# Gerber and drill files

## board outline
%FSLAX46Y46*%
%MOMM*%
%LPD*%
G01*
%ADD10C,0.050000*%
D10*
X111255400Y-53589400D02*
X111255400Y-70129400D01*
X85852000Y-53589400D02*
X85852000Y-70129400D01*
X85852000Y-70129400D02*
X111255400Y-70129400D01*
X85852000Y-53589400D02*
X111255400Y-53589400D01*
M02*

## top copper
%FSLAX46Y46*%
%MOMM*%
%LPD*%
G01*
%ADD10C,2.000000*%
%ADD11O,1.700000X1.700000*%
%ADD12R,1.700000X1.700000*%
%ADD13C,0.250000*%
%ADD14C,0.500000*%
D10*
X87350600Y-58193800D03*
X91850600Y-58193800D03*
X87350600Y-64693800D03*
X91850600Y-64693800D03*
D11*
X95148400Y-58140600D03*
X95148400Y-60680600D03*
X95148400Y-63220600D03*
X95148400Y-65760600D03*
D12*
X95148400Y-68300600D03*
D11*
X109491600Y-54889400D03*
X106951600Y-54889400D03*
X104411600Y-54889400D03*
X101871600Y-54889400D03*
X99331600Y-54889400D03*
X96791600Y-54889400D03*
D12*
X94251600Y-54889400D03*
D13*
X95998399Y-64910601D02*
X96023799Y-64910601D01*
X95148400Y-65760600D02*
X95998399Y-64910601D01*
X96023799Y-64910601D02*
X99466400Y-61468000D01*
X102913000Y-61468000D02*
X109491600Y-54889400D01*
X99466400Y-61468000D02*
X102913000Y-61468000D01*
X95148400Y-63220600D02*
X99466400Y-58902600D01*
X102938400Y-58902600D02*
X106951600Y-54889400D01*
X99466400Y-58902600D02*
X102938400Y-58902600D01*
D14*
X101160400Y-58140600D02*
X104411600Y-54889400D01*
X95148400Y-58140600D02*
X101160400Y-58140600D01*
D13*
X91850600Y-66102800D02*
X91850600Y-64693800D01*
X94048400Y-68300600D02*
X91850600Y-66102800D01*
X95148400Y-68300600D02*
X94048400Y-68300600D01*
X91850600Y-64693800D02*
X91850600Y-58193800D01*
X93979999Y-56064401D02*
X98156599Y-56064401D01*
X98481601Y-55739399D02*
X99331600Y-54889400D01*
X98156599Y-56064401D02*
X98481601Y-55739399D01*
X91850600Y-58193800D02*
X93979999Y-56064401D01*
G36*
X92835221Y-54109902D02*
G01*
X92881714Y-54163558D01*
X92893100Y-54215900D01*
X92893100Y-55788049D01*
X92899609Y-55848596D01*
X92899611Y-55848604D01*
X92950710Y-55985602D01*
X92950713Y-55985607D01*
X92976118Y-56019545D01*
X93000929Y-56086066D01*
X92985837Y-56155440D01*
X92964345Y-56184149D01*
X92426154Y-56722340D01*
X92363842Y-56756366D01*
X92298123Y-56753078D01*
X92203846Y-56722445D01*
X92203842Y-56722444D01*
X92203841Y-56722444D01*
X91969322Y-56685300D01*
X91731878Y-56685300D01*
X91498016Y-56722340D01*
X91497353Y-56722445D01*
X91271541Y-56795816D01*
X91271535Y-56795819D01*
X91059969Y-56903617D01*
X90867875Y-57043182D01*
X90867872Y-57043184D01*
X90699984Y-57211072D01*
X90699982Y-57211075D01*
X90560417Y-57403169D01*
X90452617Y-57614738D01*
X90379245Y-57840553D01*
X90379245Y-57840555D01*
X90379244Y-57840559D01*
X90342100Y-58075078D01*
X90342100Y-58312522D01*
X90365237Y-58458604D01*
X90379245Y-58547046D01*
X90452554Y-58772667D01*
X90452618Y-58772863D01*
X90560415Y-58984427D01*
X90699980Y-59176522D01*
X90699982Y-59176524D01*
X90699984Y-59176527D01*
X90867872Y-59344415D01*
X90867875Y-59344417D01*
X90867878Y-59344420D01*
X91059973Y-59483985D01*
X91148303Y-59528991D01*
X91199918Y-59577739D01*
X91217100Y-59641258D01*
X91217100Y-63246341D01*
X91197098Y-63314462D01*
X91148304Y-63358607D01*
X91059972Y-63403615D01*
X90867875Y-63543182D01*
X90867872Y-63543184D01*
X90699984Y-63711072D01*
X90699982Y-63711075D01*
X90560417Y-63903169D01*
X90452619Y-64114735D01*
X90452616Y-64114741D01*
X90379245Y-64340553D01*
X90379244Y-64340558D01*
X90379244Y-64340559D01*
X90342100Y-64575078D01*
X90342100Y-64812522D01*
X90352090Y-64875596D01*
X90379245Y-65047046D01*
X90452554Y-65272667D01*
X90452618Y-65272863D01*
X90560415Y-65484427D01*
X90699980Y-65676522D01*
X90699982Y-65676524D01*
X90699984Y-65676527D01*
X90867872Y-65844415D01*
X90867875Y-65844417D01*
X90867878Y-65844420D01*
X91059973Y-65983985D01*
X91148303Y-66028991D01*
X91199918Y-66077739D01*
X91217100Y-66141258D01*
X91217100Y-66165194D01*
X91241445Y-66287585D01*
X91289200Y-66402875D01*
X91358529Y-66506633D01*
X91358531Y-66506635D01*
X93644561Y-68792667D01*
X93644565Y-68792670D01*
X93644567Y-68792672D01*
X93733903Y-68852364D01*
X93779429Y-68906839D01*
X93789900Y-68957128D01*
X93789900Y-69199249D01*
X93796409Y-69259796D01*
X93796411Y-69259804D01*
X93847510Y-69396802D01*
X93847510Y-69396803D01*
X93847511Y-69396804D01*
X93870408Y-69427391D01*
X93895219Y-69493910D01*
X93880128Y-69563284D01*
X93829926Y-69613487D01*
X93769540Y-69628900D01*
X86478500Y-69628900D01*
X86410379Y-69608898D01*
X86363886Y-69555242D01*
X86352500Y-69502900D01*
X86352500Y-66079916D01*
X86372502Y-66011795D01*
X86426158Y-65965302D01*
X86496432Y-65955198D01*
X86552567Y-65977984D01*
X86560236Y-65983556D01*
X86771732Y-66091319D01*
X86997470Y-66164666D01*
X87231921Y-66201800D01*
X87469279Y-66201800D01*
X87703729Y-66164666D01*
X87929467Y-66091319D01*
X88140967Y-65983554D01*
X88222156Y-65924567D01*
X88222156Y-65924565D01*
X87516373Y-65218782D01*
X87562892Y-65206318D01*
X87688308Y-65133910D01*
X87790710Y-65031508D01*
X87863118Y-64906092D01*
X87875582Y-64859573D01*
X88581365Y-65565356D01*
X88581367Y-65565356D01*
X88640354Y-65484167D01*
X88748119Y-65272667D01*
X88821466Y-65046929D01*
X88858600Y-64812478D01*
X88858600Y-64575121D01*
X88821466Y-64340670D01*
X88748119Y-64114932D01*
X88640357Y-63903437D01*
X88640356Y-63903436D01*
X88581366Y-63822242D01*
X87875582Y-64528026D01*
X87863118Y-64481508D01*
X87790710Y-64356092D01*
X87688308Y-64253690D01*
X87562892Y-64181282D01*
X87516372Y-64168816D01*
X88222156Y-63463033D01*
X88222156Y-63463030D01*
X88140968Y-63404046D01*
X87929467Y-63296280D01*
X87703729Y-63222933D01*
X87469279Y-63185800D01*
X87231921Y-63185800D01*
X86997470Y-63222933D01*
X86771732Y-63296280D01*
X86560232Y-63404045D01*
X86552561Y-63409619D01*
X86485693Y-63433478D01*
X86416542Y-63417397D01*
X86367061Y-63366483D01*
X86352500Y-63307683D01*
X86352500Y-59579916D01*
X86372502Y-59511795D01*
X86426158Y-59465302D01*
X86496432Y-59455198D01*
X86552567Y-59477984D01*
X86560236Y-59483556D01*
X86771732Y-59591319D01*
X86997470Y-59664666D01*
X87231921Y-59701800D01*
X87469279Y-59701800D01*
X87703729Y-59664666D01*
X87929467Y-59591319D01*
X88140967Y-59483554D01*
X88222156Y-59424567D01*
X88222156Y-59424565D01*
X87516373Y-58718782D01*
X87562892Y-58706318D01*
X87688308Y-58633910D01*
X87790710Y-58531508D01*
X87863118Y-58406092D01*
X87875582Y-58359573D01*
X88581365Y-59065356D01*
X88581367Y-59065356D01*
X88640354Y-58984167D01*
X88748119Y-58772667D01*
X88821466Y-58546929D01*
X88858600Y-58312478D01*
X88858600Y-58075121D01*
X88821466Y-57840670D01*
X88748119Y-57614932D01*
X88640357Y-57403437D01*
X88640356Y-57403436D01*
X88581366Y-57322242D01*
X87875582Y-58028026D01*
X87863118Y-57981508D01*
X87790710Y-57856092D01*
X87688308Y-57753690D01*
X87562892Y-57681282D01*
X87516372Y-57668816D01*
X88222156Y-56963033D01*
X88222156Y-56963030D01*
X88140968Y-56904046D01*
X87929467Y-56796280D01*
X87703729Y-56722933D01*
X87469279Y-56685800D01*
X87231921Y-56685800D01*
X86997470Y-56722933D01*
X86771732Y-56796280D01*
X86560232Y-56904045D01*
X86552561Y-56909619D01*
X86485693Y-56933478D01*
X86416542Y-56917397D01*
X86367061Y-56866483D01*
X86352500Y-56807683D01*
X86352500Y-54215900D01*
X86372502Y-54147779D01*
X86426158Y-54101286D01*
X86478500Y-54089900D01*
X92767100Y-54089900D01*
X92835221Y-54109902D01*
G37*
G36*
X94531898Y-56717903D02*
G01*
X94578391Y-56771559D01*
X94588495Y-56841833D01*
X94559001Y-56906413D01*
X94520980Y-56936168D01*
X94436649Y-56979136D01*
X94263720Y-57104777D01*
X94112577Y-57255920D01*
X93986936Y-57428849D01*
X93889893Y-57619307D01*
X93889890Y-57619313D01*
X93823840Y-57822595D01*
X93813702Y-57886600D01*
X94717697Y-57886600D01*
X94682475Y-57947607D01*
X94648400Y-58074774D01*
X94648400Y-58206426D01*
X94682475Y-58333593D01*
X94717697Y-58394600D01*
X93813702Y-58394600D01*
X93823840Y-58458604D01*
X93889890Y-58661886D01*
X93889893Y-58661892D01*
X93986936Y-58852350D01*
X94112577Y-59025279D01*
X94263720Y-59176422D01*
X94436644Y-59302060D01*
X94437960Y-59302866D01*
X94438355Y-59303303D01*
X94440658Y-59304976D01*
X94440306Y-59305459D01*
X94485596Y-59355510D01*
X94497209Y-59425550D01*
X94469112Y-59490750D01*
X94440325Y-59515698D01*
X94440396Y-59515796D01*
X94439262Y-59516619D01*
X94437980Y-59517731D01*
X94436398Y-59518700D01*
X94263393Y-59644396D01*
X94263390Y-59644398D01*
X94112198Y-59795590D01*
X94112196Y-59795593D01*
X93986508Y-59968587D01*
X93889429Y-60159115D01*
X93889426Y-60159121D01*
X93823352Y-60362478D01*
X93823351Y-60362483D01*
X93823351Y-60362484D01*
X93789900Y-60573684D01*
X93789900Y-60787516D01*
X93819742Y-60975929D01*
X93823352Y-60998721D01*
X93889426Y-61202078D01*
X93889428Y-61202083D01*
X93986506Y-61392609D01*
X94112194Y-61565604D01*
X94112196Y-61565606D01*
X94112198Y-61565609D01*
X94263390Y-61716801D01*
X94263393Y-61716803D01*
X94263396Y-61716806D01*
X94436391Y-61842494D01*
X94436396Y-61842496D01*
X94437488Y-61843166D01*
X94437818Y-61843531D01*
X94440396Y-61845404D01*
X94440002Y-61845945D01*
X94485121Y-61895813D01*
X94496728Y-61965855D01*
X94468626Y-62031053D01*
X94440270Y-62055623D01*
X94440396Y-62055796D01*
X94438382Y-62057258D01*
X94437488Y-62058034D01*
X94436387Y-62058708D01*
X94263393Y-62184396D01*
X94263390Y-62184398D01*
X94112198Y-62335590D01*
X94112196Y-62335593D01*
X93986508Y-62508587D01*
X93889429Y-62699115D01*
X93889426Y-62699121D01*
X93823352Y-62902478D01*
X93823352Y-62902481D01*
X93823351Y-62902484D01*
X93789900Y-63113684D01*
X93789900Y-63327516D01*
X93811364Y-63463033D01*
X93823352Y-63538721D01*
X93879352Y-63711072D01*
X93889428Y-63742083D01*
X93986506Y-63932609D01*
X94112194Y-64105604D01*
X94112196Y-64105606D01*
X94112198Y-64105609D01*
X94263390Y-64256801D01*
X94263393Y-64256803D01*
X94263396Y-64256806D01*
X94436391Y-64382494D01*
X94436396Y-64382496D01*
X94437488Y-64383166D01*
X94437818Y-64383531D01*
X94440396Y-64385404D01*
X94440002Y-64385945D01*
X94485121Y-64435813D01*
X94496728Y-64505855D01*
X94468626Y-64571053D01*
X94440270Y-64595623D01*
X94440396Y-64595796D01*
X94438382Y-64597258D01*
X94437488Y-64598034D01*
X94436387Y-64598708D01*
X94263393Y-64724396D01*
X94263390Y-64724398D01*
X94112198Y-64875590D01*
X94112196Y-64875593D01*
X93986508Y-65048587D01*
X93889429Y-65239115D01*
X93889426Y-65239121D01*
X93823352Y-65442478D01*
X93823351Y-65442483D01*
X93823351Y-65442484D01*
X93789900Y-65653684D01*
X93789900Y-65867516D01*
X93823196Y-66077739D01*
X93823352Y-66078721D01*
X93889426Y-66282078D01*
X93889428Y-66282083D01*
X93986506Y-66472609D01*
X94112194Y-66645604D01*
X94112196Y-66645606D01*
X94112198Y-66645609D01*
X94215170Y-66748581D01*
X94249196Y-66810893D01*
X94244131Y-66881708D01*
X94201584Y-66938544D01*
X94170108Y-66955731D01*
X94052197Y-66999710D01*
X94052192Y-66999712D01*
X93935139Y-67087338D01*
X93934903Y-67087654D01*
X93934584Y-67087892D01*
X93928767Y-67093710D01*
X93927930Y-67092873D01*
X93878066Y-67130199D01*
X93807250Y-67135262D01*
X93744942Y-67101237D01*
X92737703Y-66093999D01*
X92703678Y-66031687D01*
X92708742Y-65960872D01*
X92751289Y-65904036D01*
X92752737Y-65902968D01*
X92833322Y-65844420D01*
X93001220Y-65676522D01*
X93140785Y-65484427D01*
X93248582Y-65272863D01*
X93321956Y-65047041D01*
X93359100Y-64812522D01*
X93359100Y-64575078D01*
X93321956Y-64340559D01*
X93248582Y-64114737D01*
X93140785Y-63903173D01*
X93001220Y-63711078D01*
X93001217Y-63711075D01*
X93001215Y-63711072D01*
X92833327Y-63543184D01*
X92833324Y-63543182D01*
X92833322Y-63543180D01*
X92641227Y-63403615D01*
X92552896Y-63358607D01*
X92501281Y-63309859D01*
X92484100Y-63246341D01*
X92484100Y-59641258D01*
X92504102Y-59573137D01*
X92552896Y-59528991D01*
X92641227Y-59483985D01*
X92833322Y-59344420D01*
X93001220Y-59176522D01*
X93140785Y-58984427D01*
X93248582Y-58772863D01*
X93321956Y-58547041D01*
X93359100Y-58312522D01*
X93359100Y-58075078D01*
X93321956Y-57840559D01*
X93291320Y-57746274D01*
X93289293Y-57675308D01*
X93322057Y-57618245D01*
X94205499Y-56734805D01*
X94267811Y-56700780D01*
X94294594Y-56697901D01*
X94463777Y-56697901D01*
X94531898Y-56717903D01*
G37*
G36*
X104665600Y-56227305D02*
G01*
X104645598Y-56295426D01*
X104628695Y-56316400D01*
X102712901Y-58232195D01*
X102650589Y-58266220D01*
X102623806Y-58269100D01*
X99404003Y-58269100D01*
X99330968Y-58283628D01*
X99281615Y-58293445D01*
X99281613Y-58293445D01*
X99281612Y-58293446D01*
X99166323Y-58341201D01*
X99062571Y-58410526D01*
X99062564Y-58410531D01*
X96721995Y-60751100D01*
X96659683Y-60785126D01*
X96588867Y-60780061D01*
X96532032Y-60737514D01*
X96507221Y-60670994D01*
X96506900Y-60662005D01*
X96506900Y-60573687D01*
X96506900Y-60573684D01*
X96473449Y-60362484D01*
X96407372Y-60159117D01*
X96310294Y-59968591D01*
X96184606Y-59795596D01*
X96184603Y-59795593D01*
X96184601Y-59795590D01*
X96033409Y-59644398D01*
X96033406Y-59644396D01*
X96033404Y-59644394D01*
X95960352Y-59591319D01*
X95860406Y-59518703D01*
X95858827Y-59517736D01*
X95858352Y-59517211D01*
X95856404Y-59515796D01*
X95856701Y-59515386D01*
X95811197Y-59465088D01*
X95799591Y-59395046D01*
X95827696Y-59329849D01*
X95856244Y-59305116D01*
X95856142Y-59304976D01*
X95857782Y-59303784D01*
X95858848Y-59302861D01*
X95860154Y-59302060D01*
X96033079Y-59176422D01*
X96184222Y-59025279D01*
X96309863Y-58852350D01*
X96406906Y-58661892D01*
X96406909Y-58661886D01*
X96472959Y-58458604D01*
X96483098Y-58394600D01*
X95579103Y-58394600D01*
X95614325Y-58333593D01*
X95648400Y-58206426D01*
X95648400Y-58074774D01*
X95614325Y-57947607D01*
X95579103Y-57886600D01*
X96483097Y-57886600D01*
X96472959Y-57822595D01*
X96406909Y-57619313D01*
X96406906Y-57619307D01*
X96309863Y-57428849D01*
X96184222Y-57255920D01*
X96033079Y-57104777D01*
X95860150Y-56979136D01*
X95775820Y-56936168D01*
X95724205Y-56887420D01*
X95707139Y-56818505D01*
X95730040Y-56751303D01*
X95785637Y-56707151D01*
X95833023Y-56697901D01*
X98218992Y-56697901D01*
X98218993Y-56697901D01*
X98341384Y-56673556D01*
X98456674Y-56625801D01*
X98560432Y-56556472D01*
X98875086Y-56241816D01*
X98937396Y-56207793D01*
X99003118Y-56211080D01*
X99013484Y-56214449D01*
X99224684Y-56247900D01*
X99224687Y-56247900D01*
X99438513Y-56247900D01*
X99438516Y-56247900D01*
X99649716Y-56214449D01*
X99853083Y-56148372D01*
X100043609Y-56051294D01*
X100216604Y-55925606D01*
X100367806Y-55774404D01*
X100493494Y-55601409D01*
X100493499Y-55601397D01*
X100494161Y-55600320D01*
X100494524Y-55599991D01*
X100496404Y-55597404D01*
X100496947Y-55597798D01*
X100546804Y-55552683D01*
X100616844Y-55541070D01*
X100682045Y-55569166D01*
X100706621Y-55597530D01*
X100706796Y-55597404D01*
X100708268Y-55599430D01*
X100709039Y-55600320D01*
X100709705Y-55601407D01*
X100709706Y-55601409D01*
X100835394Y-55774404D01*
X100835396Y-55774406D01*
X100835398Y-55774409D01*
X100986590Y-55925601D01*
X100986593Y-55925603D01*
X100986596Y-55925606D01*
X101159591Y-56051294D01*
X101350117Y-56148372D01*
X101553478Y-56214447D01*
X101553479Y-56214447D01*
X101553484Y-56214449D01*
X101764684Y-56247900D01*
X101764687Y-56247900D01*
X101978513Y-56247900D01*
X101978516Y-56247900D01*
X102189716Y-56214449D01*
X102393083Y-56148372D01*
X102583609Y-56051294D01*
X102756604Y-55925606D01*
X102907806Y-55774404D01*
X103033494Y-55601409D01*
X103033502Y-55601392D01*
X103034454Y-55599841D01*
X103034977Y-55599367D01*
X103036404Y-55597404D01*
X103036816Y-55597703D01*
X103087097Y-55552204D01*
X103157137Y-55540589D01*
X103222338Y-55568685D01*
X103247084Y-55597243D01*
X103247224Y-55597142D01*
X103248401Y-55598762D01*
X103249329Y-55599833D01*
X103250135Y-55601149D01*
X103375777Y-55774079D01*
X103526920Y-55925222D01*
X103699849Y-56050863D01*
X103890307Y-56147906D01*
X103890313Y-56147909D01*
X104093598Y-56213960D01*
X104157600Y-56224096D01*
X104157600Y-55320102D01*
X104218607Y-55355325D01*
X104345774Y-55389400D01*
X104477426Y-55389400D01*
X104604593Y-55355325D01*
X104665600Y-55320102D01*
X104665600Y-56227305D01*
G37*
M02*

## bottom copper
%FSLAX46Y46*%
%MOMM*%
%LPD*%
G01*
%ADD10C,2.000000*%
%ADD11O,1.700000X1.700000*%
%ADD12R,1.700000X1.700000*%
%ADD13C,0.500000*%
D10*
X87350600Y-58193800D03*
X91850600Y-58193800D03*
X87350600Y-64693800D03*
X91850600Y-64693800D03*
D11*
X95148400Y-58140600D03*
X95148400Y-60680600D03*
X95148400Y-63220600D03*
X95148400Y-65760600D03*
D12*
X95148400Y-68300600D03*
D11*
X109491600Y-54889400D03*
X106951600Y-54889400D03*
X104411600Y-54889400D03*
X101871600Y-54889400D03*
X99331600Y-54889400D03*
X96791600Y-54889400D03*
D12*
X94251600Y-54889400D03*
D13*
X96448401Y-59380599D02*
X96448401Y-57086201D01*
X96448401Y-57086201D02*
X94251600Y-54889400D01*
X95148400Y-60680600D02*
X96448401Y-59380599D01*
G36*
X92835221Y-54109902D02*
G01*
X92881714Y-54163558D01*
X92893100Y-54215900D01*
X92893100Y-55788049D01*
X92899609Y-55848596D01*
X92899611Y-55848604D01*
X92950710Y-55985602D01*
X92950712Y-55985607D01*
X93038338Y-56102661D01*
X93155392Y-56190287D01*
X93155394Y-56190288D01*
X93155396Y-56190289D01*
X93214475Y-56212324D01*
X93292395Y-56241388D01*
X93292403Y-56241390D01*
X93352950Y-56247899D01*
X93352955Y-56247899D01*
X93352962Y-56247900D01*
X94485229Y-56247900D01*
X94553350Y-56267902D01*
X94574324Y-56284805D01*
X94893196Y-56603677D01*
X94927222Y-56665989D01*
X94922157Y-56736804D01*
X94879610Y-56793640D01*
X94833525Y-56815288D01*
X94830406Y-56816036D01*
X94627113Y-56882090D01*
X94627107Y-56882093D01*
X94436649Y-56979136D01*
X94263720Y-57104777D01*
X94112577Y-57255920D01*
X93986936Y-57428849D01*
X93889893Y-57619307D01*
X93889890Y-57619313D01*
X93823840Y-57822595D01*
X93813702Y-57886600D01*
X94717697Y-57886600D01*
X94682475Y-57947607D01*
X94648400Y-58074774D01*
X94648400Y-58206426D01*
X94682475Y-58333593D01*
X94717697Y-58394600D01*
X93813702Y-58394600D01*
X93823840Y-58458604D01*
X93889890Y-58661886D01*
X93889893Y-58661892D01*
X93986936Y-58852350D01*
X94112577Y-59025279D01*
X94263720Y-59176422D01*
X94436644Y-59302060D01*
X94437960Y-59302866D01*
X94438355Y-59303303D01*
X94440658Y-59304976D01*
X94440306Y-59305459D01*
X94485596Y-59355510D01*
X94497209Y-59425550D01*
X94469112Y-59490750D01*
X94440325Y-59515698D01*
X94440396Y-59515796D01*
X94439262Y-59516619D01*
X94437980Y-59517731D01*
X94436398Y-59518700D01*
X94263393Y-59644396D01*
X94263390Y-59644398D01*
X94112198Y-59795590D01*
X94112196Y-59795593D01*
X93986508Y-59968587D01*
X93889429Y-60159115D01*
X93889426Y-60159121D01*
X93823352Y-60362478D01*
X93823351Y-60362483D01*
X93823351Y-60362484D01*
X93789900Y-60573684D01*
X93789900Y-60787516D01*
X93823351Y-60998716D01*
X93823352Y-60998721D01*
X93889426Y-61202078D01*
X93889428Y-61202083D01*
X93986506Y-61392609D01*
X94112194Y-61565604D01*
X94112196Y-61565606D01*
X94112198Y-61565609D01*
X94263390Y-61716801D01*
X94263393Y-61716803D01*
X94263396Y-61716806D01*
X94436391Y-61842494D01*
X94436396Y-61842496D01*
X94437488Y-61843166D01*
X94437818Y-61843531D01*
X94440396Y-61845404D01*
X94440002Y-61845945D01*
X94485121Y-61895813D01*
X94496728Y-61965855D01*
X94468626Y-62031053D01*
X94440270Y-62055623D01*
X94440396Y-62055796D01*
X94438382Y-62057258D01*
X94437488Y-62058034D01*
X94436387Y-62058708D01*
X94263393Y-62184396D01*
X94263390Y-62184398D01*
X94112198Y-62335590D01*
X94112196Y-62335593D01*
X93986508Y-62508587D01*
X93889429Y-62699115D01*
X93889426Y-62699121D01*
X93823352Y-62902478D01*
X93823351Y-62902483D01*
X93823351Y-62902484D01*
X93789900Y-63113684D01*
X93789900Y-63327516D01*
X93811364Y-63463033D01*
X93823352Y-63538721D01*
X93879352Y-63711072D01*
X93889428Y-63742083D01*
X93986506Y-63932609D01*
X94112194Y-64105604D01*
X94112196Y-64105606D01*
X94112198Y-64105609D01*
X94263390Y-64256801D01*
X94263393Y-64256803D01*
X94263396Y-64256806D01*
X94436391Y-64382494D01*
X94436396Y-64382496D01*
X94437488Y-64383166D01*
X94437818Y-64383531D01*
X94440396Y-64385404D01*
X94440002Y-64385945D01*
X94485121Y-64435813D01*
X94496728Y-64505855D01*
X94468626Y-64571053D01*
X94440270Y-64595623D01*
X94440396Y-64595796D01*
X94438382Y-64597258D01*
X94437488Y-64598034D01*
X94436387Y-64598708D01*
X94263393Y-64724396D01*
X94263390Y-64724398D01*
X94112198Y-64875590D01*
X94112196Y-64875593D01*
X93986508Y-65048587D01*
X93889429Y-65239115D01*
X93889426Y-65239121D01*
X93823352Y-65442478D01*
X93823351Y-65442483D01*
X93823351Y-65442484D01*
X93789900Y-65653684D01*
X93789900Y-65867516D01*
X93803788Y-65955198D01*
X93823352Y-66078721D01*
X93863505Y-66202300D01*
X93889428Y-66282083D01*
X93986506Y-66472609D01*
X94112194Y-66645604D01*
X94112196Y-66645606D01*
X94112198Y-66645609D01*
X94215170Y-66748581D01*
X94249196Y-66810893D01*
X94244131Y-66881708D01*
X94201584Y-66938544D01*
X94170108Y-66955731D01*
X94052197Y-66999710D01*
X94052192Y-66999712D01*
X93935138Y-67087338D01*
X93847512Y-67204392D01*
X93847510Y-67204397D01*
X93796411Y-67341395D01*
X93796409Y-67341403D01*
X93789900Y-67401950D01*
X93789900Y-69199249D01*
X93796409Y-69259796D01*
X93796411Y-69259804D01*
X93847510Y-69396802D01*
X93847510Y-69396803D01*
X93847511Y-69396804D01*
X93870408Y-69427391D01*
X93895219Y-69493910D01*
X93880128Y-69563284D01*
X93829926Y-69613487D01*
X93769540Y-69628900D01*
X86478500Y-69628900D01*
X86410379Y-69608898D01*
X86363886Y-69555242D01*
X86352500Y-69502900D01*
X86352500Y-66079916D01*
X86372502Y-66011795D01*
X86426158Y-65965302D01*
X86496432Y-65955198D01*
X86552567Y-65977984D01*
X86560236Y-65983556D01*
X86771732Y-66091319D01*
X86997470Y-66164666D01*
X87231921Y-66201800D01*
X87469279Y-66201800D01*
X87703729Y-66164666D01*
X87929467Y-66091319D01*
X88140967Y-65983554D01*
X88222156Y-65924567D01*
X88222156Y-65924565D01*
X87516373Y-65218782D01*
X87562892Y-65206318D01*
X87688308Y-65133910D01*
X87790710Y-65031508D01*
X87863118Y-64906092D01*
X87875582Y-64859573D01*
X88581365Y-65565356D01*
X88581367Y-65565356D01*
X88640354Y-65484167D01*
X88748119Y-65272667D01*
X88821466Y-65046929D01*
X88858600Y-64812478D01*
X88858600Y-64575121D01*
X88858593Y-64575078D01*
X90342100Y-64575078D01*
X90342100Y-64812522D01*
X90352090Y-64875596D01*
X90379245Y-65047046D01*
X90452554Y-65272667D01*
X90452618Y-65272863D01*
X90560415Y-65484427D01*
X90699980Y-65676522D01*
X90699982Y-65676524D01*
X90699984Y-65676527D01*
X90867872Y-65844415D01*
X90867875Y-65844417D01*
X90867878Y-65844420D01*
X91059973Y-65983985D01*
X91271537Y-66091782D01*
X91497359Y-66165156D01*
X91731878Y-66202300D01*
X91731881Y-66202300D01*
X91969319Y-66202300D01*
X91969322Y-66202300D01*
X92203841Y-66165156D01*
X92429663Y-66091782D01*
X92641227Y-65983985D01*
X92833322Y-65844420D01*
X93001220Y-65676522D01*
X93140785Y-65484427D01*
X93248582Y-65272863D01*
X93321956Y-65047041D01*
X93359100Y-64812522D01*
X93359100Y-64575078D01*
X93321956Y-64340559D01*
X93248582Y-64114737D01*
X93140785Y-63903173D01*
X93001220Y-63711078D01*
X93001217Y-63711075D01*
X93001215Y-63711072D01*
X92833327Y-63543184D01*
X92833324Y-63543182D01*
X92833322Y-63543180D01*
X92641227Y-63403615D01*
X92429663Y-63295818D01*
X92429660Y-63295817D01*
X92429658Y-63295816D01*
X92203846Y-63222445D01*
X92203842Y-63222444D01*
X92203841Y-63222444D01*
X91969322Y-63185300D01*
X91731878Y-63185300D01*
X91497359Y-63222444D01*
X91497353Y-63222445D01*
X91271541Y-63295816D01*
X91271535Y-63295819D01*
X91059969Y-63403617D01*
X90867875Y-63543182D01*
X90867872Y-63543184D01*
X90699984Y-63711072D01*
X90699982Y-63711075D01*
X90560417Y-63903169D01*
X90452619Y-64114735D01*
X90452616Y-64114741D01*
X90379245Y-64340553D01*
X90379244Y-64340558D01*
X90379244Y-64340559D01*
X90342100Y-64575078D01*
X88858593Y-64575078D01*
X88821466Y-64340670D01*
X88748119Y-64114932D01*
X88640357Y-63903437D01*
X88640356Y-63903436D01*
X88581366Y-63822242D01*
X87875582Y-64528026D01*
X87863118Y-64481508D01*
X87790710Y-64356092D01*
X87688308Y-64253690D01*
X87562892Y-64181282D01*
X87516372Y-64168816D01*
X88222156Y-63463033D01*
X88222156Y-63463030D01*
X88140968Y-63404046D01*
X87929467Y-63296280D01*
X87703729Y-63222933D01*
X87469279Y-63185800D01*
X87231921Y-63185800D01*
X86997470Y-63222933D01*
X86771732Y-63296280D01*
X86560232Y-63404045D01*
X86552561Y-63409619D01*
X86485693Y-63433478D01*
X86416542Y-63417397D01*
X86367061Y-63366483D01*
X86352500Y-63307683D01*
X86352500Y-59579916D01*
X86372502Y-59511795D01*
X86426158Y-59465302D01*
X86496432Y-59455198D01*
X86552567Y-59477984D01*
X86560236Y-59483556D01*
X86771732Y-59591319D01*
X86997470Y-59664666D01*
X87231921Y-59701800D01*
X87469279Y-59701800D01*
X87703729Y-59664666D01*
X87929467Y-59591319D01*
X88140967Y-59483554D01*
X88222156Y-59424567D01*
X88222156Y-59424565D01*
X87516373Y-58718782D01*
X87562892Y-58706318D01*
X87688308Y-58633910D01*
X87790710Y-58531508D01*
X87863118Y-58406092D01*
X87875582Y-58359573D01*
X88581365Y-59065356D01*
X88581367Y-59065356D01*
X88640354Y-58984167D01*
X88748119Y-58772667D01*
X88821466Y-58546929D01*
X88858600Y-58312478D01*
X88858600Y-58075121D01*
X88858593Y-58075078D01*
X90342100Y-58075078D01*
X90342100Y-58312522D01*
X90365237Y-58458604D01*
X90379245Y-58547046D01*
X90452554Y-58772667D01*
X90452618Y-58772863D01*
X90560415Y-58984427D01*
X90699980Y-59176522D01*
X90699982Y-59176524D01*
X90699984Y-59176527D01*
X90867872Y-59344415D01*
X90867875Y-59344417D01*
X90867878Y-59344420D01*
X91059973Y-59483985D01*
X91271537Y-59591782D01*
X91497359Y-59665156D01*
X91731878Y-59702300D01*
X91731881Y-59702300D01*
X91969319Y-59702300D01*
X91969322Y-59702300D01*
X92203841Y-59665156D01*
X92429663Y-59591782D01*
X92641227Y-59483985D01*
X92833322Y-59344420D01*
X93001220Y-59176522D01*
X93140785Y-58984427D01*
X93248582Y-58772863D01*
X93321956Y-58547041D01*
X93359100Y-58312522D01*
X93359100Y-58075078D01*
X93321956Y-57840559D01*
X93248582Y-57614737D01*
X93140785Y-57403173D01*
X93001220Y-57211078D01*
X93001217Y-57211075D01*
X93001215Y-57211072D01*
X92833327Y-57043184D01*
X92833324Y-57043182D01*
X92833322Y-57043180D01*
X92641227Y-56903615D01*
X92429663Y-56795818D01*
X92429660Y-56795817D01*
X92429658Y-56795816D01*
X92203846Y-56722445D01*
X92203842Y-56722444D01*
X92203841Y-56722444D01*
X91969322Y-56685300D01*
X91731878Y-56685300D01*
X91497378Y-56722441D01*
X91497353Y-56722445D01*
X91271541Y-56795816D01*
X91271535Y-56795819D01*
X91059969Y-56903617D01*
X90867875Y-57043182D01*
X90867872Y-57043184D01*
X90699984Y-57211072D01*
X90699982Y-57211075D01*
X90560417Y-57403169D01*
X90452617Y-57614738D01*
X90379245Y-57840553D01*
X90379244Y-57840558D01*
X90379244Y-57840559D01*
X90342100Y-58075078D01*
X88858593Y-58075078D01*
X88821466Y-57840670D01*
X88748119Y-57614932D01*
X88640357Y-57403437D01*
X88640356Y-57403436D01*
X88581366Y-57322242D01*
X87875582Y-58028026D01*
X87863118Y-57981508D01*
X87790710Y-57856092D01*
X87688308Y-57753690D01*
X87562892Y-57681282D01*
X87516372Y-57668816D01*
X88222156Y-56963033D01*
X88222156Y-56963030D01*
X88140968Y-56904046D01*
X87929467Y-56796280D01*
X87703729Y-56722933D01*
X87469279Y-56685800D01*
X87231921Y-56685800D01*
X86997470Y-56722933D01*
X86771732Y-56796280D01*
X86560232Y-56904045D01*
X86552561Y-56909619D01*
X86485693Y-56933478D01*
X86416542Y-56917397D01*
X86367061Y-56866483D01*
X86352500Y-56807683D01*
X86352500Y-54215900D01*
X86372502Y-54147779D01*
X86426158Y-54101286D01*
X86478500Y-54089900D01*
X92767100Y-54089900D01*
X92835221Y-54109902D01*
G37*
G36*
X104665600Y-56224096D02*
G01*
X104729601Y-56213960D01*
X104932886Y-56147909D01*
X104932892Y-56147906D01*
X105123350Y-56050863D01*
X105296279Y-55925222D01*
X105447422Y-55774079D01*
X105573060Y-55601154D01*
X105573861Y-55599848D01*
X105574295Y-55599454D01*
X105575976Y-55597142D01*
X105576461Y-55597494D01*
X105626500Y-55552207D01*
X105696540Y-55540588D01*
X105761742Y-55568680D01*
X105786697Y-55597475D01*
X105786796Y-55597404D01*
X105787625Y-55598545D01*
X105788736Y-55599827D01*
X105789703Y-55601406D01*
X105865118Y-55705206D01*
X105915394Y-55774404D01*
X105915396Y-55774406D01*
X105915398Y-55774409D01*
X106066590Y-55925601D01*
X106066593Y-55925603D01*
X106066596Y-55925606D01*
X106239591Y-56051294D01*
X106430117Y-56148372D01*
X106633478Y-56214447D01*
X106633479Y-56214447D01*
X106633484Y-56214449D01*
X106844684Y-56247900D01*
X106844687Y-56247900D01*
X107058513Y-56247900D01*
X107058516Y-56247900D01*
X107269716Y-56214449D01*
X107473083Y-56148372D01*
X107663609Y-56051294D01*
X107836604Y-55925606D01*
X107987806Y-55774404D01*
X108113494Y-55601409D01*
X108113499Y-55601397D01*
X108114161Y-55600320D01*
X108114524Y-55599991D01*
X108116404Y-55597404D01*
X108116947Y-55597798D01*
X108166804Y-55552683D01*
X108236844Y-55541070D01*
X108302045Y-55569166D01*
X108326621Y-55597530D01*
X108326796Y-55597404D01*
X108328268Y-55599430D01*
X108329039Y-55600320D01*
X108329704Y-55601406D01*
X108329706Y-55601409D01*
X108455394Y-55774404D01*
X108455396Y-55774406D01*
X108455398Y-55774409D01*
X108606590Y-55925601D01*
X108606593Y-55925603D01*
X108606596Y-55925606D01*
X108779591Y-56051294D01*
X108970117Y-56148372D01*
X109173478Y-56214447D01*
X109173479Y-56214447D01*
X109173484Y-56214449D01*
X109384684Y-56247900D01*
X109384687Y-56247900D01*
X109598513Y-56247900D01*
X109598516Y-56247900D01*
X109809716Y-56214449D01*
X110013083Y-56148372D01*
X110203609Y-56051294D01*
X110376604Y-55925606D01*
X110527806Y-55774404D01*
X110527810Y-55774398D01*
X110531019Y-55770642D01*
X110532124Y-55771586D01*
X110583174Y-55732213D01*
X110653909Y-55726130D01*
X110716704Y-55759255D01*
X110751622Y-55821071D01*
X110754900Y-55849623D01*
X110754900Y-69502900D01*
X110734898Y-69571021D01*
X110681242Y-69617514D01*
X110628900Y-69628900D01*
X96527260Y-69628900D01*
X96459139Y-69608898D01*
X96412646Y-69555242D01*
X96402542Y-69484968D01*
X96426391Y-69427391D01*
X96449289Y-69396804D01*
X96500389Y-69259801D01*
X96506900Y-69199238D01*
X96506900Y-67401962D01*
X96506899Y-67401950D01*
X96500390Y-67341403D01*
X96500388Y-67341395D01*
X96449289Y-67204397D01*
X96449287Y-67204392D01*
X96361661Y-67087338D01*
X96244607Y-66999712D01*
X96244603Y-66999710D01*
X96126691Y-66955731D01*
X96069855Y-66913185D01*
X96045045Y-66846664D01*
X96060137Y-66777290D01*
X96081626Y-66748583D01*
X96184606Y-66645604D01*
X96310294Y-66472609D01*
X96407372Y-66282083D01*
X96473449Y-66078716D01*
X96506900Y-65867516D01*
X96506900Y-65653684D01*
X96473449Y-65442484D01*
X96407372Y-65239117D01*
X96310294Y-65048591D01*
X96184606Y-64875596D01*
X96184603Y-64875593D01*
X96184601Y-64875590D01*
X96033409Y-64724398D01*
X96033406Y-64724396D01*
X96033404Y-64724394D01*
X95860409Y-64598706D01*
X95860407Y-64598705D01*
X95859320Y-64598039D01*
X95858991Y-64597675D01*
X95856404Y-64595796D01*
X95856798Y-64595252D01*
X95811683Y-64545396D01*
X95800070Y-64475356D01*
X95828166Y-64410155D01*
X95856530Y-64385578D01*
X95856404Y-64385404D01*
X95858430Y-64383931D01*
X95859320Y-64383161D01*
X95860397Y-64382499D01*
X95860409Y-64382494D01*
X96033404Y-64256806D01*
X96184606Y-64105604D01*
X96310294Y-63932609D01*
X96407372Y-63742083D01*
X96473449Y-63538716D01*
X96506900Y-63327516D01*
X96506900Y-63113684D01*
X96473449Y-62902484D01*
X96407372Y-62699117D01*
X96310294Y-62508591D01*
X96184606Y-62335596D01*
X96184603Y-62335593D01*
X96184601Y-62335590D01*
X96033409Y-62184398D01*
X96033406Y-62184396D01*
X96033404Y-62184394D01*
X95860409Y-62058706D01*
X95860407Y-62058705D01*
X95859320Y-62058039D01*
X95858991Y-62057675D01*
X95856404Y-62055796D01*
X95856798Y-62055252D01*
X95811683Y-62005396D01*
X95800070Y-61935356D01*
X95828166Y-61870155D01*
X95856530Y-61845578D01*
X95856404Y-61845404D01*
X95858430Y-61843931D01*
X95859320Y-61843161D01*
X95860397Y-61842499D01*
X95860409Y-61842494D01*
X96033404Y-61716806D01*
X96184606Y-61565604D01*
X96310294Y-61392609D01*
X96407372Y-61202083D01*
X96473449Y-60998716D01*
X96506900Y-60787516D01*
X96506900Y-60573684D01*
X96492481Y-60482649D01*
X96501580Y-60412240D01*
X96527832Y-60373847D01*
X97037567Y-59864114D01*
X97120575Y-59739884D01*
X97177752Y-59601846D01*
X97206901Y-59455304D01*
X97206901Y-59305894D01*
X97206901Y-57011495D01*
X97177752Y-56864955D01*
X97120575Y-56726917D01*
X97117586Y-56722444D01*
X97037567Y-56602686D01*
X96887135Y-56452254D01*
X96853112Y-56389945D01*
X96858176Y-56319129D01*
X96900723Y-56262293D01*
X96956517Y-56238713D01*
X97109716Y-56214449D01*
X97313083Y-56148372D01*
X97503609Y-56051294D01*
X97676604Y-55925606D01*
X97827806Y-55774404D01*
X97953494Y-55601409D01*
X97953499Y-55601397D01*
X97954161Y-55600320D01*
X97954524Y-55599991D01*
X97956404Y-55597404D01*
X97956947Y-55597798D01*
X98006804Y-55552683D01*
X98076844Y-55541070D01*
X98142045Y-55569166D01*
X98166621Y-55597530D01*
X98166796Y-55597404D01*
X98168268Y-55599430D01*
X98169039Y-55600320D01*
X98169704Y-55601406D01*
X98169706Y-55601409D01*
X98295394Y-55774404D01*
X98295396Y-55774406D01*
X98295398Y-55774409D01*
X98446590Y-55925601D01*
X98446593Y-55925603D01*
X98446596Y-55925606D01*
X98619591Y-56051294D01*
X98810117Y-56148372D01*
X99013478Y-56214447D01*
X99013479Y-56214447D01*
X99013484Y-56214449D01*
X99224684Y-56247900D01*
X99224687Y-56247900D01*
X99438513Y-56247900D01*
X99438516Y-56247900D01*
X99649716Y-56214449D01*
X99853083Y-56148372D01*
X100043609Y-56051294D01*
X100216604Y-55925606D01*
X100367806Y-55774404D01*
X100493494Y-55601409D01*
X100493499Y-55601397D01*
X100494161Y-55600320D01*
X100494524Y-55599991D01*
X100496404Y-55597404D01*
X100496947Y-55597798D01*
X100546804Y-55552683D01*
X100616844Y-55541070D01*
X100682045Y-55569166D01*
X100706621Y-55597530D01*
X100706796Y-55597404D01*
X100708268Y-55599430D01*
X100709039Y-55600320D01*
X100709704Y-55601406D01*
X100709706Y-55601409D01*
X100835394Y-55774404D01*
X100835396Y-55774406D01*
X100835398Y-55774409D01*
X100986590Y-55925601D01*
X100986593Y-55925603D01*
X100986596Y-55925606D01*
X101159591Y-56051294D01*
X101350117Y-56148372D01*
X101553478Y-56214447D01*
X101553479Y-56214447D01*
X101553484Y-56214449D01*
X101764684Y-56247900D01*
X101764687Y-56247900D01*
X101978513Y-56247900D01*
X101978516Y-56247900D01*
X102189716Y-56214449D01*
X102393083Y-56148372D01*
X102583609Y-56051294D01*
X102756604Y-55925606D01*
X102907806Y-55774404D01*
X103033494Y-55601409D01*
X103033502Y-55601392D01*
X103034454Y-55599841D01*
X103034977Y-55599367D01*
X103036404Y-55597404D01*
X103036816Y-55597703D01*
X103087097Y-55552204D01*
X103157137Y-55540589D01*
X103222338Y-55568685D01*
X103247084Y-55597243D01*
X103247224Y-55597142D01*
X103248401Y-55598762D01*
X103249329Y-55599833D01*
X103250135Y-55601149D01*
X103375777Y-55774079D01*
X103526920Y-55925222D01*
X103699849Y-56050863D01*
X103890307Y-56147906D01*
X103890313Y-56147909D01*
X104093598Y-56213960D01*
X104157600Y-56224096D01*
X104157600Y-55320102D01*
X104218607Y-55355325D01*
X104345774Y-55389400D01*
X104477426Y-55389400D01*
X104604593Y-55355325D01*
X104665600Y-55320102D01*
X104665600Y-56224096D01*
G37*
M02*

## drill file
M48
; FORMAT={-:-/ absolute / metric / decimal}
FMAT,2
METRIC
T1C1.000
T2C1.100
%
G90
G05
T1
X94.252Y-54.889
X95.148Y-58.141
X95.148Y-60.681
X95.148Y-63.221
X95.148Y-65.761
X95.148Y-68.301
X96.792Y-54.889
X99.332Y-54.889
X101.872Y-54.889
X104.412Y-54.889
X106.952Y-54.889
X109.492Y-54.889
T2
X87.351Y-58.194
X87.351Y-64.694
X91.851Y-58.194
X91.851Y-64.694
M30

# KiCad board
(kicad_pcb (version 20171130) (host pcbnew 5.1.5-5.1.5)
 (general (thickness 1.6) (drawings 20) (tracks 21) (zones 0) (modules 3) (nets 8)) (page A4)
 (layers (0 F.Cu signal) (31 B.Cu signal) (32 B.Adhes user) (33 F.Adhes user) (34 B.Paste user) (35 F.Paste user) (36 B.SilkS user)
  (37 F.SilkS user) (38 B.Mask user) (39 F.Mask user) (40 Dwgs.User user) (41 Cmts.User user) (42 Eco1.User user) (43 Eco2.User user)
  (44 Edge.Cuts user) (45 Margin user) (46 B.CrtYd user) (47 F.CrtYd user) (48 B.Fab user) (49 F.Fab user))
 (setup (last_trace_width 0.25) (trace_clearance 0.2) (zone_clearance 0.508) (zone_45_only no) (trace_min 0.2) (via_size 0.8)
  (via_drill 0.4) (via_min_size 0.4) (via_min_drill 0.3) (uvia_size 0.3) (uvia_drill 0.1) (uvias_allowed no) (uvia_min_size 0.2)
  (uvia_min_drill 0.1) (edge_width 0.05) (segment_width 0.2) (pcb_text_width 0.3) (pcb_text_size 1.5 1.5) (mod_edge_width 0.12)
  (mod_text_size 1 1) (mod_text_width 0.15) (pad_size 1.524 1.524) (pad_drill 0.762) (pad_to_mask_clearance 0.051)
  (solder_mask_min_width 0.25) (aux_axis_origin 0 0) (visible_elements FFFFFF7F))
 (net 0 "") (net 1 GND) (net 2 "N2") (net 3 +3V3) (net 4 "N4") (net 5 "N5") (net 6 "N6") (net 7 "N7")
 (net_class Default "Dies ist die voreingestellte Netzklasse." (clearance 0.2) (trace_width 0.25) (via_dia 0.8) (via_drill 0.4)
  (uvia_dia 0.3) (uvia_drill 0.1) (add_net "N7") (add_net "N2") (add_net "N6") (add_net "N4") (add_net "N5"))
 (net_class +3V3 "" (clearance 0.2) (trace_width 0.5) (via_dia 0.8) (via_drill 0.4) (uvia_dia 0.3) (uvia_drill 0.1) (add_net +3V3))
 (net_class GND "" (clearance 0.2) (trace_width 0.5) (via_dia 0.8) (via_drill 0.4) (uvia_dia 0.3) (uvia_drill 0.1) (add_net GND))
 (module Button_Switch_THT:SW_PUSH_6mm (layer F.Cu) (at 87.3506 64.6938 90)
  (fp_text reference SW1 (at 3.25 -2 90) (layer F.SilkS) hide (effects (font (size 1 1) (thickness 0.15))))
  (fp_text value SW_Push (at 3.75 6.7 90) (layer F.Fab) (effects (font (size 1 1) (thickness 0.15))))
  (pad 1 thru_hole circle (at 6.5 0 180) (size 2 2) (drill 1.1) (layers *.Cu *.Mask) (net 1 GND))
  (pad 2 thru_hole circle (at 6.5 4.5 180) (size 2 2) (drill 1.1) (layers *.Cu *.Mask) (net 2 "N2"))
  (pad 1 thru_hole circle (at 0 0 180) (size 2 2) (drill 1.1) (layers *.Cu *.Mask) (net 1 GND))
  (pad 2 thru_hole circle (at 0 4.5 180) (size 2 2) (drill 1.1) (layers *.Cu *.Mask) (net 2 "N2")))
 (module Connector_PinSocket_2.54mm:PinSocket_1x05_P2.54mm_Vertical (layer F.Cu) (at 95.1484 68.3006 180)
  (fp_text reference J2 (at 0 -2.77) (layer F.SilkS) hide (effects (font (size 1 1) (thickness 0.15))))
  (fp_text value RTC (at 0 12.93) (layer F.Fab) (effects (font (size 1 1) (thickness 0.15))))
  (pad 5 thru_hole oval (at 0 10.16 180) (size 1.7 1.7) (drill 1) (layers *.Cu *.Mask) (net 1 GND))
  (pad 4 thru_hole oval (at 0 7.62 180) (size 1.7 1.7) (drill 1) (layers *.Cu *.Mask) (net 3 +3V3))
  (pad 3 thru_hole oval (at 0 5.08 180) (size 1.7 1.7) (drill 1) (layers *.Cu *.Mask) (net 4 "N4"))
  (pad 2 thru_hole oval (at 0 2.54 180) (size 1.7 1.7) (drill 1) (layers *.Cu *.Mask) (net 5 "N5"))
  (pad 1 thru_hole rect (at 0 0 180) (size 1.7 1.7) (drill 1) (layers *.Cu *.Mask) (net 2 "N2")))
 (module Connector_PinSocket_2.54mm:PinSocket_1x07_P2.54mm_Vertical (layer B.Cu) (at 94.2516 54.8894 270)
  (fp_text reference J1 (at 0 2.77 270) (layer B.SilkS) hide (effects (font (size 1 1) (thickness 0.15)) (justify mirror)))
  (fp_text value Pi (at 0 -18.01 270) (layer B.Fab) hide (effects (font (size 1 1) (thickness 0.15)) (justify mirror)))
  (pad 7 thru_hole oval (at 0 -15.24 270) (size 1.7 1.7) (drill 1) (layers *.Cu *.Mask) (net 5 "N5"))
  (pad 6 thru_hole oval (at 0 -12.7 270) (size 1.7 1.7) (drill 1) (layers *.Cu *.Mask) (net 4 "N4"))
  (pad 5 thru_hole oval (at 0 -10.16 270) (size 1.7 1.7) (drill 1) (layers *.Cu *.Mask) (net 1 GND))
  (pad 4 thru_hole oval (at 0 -7.62 270) (size 1.7 1.7) (drill 1) (layers *.Cu *.Mask) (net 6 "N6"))
  (pad 3 thru_hole oval (at 0 -5.08 270) (size 1.7 1.7) (drill 1) (layers *.Cu *.Mask) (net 2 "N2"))
  (pad 2 thru_hole oval (at 0 -2.54 270) (size 1.7 1.7) (drill 1) (layers *.Cu *.Mask) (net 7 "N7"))
  (pad 1 thru_hole rect (at 0 0 270) (size 1.7 1.7) (drill 1) (layers *.Cu *.Mask) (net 3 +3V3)))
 (gr_line (start 111.2554 53.5894) (end 111.2554 70.1294) (layer Edge.Cuts) (width 0.05))
 (gr_line (start 85.852 53.5894) (end 85.852 70.1294) (layer Edge.Cuts) (width 0.05))
 (gr_line (start 85.852 70.1294) (end 111.2554 70.1294) (layer Edge.Cuts) (width 0.05))
 (gr_line (start 85.852 53.5894) (end 111.2554 53.5894) (layer Edge.Cuts) (width 0.05))
 (segment (start 95.998399 64.910601) (end 96.023799 64.910601) (width 0.25) (layer F.Cu) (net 5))
 (segment (start 95.1484 65.7606) (end 95.998399 64.910601) (width 0.25) (layer F.Cu) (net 5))
 (segment (start 96.023799 64.910601) (end 99.4664 61.468) (width 0.25) (layer F.Cu) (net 5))
 (segment (start 102.913 61.468) (end 109.4916 54.8894) (width 0.25) (layer F.Cu) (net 5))
 (segment (start 99.4664 61.468) (end 102.913 61.468) (width 0.25) (layer F.Cu) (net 5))
 (segment (start 95.1484 63.2206) (end 99.4664 58.9026) (width 0.25) (layer F.Cu) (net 4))
 (segment (start 102.9384 58.9026) (end 106.9516 54.8894) (width 0.25) (layer F.Cu) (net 4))
 (segment (start 99.4664 58.9026) (end 102.9384 58.9026) (width 0.25) (layer F.Cu) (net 4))
 (segment (start 101.1604 58.1406) (end 104.4116 54.8894) (width 0.5) (layer F.Cu) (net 1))
 (segment (start 95.1484 58.1406) (end 101.1604 58.1406) (width 0.5) (layer F.Cu) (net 1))
 (segment (start 91.8506 66.1028) (end 91.8506 64.6938) (width 0.25) (layer F.Cu) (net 2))
 (segment (start 94.0484 68.3006) (end 91.8506 66.1028) (width 0.25) (layer F.Cu) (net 2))
 (segment (start 95.1484 68.3006) (end 94.0484 68.3006) (width 0.25) (layer F.Cu) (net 2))
 (segment (start 91.8506 64.6938) (end 91.8506 58.1938) (width 0.25) (layer F.Cu) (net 2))
 (segment (start 93.979999 56.064401) (end 98.156599 56.064401) (width 0.25) (layer F.Cu) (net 2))
 (segment (start 98.481601 55.739399) (end 99.3316 54.8894) (width 0.25) (layer F.Cu) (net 2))
 (segment (start 98.156599 56.064401) (end 98.481601 55.739399) (width 0.25) (layer F.Cu) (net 2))
 (segment (start 91.8506 58.1938) (end 93.979999 56.064401) (width 0.25) (layer F.Cu) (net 2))
 (segment (start 96.448401 59.380599) (end 96.448401 57.086201) (width 0.5) (layer B.Cu) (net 3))
 (segment (start 96.448401 57.086201) (end 94.2516 54.8894) (width 0.5) (layer B.Cu) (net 3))
 (segment (start 95.1484 60.6806) (end 96.448401 59.380599) (width 0.5) (layer B.Cu) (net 3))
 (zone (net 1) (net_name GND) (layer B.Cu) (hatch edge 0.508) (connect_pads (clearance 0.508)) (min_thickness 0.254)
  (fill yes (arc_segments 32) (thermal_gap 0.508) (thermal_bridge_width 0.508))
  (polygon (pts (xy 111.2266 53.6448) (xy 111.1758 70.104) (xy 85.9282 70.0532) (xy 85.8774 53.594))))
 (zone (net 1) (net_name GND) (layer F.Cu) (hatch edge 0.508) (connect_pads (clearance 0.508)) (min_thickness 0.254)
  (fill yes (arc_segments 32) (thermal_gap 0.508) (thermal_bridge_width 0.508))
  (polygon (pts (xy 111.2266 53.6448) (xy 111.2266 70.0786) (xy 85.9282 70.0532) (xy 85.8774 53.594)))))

